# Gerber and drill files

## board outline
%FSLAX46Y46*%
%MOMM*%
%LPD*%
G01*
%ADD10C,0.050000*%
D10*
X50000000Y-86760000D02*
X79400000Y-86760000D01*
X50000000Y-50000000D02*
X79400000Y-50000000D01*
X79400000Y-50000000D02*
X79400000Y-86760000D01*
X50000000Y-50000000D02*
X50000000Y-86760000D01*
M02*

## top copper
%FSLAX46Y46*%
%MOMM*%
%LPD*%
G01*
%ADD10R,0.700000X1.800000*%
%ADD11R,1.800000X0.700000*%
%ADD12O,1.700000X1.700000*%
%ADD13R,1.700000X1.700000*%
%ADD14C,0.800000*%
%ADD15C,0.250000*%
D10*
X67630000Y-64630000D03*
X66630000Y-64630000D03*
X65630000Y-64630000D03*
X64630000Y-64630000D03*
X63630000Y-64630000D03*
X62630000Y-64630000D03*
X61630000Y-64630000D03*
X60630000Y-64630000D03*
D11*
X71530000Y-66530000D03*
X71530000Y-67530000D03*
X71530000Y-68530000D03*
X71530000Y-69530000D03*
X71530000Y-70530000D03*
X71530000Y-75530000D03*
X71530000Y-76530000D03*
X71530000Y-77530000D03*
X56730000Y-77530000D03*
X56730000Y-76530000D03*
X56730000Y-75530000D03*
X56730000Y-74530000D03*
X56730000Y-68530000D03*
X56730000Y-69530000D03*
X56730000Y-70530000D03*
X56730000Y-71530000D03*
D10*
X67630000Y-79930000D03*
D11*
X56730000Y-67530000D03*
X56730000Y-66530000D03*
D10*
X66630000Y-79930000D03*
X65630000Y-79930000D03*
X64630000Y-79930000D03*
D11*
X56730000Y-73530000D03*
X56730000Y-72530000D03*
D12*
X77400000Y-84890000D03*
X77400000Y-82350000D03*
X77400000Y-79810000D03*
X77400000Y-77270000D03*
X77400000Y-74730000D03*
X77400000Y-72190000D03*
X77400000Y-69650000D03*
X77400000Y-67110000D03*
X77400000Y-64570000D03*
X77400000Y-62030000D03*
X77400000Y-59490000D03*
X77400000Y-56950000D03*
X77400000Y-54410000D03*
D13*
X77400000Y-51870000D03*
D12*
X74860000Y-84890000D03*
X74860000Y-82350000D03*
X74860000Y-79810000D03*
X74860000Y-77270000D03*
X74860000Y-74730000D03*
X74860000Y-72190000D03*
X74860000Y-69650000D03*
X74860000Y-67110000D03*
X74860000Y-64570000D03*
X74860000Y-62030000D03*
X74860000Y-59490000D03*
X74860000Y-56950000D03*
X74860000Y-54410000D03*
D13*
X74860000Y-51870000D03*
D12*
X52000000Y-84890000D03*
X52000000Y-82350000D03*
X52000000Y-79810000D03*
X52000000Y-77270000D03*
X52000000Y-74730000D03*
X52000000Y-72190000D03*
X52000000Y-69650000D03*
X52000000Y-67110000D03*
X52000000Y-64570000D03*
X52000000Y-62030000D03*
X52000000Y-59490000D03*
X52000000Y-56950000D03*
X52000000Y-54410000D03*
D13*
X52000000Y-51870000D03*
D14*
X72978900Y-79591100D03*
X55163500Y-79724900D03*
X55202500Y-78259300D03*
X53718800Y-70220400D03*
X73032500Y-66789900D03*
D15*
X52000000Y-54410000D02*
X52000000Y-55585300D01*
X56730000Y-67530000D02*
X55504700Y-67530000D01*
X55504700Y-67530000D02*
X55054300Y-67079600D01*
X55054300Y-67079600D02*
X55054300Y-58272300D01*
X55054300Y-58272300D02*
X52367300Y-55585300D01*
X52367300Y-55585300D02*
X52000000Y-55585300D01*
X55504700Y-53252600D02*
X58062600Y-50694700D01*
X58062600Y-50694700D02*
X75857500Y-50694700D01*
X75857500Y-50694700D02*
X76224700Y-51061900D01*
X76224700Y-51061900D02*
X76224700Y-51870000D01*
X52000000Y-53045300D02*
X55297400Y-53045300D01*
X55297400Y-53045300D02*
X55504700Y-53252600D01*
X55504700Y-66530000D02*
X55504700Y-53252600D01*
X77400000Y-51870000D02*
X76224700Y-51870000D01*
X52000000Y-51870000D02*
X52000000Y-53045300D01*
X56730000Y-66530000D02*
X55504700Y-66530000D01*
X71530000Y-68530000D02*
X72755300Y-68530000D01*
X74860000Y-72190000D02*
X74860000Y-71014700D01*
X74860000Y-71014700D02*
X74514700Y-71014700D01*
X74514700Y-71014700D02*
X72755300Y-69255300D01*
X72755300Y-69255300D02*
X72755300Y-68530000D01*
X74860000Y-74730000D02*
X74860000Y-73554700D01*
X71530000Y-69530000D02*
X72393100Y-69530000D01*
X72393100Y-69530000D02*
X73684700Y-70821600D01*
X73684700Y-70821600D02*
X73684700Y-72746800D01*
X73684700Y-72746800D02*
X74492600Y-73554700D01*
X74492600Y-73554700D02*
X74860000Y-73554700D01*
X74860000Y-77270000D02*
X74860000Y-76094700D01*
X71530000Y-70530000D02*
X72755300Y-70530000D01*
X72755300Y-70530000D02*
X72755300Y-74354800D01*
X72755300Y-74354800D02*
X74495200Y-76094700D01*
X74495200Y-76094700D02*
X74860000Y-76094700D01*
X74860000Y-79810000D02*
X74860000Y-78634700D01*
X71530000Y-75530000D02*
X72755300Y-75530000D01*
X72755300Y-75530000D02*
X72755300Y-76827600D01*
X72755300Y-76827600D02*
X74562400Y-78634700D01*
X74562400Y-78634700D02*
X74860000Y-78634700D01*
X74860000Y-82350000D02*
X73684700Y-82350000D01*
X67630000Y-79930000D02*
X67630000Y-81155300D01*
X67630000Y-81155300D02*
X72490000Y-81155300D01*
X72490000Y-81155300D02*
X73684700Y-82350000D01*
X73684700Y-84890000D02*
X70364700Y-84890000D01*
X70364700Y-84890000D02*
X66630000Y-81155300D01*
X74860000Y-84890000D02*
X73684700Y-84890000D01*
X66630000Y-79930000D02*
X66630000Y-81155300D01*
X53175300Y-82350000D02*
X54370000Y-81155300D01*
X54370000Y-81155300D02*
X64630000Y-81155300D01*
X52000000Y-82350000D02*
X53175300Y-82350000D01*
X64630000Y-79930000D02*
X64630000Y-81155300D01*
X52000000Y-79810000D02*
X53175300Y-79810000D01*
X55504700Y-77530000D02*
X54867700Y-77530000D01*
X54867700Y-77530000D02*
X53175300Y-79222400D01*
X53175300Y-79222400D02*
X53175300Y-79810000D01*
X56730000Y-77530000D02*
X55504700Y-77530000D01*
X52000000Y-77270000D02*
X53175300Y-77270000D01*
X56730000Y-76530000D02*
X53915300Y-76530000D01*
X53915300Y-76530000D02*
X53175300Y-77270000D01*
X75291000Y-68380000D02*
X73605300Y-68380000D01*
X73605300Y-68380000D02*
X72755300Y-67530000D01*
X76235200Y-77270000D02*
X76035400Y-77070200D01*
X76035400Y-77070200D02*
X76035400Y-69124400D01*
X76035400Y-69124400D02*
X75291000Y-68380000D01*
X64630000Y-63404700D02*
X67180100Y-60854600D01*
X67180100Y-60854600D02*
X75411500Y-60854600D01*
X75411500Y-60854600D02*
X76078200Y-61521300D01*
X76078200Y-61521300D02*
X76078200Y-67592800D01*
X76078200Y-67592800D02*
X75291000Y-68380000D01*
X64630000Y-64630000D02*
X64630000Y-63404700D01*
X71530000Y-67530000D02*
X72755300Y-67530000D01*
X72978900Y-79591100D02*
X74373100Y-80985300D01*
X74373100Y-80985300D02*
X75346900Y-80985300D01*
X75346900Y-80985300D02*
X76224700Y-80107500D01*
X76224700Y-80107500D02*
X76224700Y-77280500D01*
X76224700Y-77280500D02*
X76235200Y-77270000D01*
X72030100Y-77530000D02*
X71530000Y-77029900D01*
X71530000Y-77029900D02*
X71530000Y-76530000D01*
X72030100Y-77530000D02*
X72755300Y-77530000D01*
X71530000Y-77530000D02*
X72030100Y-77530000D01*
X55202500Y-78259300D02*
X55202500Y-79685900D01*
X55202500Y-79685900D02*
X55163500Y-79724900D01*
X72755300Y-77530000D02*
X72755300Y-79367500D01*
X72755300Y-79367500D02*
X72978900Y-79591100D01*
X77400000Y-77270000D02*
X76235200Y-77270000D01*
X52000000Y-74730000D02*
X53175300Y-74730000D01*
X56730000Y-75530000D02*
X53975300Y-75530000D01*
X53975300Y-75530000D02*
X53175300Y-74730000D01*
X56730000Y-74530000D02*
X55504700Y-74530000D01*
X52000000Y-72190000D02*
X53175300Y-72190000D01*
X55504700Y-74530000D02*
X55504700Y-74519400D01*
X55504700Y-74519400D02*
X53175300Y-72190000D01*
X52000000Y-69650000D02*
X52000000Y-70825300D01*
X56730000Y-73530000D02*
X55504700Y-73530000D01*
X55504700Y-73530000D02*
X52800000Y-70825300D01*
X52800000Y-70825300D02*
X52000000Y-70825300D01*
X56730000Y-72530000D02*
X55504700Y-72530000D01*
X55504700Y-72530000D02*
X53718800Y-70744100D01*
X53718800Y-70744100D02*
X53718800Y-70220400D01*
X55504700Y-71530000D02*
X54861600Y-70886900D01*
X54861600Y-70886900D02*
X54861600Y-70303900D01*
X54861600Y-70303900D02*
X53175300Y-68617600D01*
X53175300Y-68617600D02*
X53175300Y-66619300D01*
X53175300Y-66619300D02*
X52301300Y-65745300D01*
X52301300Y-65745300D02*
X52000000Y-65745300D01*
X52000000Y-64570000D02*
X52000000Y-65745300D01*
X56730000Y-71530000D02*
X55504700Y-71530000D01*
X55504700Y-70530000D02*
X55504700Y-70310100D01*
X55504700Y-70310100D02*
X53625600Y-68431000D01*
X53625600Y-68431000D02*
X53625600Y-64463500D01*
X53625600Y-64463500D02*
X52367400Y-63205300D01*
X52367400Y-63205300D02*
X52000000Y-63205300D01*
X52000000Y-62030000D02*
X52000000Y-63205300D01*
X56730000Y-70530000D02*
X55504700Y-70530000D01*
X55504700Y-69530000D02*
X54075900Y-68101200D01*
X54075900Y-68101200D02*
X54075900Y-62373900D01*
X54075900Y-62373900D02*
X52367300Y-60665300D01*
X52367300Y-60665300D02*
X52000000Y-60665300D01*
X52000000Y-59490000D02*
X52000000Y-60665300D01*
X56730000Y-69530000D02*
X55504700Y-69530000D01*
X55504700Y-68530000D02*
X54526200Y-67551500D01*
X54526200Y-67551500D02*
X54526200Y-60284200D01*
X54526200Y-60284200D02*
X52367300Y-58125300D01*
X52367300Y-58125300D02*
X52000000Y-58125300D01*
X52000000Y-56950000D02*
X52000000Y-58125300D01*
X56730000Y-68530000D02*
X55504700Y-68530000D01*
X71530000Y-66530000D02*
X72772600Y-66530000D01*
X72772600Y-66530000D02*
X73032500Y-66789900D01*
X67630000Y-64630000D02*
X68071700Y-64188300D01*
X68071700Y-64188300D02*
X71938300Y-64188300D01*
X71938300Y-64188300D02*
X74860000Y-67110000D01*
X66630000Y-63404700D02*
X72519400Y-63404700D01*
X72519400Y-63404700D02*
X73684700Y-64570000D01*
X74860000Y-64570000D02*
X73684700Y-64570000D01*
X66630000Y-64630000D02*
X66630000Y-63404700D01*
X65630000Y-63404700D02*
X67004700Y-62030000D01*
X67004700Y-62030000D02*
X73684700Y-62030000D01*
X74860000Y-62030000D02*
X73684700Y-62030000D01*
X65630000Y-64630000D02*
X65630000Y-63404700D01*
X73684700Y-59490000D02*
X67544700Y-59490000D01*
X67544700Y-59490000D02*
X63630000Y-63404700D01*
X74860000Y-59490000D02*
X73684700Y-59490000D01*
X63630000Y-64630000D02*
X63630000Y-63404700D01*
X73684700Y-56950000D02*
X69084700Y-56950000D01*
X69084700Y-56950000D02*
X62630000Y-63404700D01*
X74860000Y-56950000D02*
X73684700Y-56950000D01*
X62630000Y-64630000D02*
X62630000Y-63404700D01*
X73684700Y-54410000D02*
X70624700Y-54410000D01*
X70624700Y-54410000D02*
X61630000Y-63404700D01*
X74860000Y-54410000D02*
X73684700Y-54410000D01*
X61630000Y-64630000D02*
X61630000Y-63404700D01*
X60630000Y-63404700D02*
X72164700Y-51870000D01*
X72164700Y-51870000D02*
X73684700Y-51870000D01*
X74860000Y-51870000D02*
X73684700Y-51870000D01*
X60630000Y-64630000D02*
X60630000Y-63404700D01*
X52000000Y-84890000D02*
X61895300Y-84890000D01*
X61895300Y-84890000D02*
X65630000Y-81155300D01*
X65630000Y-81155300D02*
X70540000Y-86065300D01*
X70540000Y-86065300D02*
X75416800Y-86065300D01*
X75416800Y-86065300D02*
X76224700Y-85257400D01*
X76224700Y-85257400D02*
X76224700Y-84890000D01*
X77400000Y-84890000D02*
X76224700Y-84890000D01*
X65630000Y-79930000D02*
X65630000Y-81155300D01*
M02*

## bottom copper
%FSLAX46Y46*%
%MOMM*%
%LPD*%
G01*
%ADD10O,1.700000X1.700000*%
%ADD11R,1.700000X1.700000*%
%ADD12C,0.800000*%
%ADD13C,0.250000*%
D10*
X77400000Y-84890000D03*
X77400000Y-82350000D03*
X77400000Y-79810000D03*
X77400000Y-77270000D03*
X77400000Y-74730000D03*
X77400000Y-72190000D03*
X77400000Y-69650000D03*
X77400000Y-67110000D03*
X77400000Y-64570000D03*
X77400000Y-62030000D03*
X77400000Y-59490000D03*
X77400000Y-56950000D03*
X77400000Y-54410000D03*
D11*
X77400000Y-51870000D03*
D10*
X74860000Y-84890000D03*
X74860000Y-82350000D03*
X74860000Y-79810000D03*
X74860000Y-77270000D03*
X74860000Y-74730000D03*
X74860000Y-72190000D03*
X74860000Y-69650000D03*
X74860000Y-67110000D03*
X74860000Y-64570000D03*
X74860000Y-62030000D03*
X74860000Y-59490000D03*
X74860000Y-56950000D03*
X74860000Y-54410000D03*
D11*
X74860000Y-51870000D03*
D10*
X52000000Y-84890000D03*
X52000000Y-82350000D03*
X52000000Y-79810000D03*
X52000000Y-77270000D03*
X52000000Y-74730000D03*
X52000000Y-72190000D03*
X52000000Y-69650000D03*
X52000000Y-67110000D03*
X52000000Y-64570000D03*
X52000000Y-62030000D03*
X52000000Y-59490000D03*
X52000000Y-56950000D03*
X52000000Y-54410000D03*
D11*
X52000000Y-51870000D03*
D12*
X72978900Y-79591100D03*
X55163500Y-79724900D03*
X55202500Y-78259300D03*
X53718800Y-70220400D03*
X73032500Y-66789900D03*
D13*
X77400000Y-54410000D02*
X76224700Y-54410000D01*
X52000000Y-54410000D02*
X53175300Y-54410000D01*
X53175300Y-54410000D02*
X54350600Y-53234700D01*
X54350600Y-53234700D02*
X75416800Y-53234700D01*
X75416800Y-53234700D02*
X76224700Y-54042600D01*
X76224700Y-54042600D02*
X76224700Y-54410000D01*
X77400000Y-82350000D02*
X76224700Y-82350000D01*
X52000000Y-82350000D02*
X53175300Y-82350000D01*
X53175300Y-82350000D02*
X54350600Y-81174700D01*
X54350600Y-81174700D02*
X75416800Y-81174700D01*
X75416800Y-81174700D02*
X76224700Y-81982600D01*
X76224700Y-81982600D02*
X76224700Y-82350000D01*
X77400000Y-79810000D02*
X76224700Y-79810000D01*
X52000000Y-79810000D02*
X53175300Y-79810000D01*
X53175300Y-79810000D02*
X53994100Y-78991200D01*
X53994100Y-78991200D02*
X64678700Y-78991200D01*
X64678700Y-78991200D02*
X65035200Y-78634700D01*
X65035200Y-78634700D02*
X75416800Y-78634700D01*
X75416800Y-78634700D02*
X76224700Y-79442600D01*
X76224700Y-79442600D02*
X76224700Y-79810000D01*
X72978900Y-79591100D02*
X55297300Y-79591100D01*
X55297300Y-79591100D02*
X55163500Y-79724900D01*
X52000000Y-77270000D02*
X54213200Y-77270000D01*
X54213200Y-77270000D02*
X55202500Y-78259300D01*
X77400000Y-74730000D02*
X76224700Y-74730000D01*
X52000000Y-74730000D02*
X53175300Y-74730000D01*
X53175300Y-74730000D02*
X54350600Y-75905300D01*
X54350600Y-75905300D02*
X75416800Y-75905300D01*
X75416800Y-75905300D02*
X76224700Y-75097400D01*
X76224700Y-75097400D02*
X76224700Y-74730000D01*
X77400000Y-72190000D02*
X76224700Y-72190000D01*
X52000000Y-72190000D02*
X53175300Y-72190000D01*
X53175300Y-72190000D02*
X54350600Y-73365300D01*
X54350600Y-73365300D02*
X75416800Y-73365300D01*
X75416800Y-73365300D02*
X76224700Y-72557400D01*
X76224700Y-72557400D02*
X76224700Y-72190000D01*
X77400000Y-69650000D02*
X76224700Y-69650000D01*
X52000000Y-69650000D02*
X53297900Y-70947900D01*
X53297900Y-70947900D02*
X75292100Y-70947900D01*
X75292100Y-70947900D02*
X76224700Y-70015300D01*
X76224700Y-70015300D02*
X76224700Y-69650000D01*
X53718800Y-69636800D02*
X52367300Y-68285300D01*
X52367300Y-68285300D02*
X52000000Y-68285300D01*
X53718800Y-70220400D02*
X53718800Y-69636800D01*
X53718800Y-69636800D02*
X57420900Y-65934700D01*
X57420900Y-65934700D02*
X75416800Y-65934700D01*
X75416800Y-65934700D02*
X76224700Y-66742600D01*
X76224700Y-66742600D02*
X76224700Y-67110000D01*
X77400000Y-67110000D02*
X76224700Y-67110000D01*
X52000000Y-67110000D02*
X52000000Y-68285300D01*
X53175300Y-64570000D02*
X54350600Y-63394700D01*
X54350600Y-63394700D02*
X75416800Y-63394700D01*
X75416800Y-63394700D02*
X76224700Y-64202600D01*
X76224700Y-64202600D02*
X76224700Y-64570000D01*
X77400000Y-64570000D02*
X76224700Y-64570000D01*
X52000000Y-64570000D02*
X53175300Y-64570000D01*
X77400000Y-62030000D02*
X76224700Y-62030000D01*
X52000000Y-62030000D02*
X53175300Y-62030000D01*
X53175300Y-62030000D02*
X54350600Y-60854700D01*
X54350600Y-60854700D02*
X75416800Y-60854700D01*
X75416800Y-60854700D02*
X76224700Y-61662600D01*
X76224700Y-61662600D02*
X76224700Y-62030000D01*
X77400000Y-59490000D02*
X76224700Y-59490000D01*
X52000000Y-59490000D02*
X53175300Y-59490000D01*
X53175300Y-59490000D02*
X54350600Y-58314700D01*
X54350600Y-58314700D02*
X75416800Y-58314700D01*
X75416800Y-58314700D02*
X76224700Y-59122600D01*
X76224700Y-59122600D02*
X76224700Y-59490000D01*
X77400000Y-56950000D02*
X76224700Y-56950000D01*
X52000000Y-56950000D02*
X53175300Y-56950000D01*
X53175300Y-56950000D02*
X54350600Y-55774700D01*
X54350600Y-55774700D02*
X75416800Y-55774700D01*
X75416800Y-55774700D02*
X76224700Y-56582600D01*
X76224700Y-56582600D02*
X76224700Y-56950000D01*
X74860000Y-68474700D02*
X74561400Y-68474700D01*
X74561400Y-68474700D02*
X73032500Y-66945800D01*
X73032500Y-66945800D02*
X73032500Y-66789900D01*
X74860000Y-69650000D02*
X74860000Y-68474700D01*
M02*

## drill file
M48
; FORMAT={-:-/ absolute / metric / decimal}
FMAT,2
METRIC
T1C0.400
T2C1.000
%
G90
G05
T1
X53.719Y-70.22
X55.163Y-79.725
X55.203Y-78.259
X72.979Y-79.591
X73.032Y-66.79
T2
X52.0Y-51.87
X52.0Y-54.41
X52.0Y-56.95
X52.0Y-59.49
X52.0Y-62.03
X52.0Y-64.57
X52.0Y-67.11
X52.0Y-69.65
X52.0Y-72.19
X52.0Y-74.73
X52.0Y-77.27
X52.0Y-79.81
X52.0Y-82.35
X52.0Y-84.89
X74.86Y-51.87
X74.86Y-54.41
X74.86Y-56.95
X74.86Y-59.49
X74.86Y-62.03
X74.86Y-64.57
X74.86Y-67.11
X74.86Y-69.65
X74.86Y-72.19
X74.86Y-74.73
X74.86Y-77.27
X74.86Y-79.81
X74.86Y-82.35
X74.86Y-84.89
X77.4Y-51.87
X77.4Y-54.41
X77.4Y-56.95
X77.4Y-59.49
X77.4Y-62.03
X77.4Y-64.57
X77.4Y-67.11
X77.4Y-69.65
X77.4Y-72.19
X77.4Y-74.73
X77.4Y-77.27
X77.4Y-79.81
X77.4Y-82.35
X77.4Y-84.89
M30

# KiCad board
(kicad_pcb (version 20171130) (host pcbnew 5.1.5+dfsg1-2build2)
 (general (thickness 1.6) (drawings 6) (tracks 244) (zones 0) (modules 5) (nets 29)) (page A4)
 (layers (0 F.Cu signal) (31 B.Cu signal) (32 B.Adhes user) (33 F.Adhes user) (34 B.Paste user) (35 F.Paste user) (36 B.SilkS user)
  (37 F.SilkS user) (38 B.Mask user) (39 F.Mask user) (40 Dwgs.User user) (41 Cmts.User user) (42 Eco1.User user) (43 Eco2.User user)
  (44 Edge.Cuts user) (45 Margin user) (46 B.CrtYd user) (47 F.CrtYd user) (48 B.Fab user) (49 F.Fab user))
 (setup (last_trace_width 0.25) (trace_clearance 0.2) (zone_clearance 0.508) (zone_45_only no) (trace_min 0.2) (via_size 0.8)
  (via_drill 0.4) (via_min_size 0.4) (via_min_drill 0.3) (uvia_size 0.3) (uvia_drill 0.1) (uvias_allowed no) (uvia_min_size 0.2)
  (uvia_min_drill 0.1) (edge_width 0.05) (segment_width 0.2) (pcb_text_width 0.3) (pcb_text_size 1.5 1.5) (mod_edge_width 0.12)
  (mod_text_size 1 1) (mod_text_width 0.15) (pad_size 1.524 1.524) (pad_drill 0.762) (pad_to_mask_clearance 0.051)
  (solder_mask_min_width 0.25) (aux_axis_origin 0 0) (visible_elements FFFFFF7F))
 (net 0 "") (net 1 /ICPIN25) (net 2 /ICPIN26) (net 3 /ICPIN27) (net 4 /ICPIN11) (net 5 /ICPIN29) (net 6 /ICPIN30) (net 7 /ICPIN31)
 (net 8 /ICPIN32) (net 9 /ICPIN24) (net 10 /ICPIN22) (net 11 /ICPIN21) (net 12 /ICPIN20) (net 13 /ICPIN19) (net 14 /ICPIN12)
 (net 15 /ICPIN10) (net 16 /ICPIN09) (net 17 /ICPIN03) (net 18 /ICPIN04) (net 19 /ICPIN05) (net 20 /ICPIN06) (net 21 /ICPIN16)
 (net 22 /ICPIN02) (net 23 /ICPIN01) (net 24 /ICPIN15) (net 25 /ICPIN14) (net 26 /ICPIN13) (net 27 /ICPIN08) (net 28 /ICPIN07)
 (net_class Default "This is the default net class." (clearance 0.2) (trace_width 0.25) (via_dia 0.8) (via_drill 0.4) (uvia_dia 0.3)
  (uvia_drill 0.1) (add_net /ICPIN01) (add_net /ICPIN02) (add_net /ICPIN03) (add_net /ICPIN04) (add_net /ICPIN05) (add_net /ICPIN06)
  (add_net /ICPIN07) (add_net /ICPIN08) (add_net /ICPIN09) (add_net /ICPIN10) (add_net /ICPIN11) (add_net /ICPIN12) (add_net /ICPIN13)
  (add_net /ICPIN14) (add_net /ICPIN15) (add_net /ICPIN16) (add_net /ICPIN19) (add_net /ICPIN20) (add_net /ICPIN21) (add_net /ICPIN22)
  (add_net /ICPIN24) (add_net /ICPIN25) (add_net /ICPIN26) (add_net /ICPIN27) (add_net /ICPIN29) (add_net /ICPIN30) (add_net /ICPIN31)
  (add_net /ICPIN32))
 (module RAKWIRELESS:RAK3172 (layer F.Cu) (at 64.13 72.28)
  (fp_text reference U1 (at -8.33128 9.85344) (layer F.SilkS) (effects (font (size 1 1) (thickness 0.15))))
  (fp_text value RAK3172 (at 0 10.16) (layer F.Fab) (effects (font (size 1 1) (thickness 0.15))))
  (pad 25 smd rect (at 3.5 -7.65 270) (size 1.8 0.7) (layers F.Cu F.Paste F.Mask) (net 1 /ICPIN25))
  (pad 26 smd rect (at 2.5 -7.65 270) (size 1.8 0.7) (layers F.Cu F.Paste F.Mask) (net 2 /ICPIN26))
  (pad 27 smd rect (at 1.5 -7.65 270) (size 1.8 0.7) (layers F.Cu F.Paste F.Mask) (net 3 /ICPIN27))
  (pad 28 smd rect (at 0.5 -7.65 270) (size 1.8 0.7) (layers F.Cu F.Paste F.Mask) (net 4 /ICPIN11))
  (pad 29 smd rect (at -0.5 -7.65 270) (size 1.8 0.7) (layers F.Cu F.Paste F.Mask) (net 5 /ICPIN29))
  (pad 30 smd rect (at -1.5 -7.65 270) (size 1.8 0.7) (layers F.Cu F.Paste F.Mask) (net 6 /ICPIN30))
  (pad 31 smd rect (at -2.5 -7.65 270) (size 1.8 0.7) (layers F.Cu F.Paste F.Mask) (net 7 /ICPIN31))
  (pad 32 smd rect (at -3.5 -7.65 270) (size 1.8 0.7) (layers F.Cu F.Paste F.Mask) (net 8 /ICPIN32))
  (pad 24 smd rect (at 7.4 -5.75) (size 1.8 0.7) (layers F.Cu F.Paste F.Mask) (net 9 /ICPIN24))
  (pad 23 smd rect (at 7.4 -4.75) (size 1.8 0.7) (layers F.Cu F.Paste F.Mask) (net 4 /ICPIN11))
  (pad 22 smd rect (at 7.4 -3.75) (size 1.8 0.7) (layers F.Cu F.Paste F.Mask) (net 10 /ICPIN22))
  (pad 21 smd rect (at 7.4 -2.75) (size 1.8 0.7) (layers F.Cu F.Paste F.Mask) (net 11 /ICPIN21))
  (pad 20 smd rect (at 7.4 -1.75) (size 1.8 0.7) (layers F.Cu F.Paste F.Mask) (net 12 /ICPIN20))
  (pad 19 smd rect (at 7.4 3.25) (size 1.8 0.7) (layers F.Cu F.Paste F.Mask) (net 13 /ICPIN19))
  (pad 18 smd rect (at 7.4 4.25) (size 1.8 0.7) (layers F.Cu F.Paste F.Mask) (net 4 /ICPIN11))
  (pad 17 smd rect (at 7.4 5.25) (size 1.8 0.7) (layers F.Cu F.Paste F.Mask) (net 4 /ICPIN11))
  (pad 12 smd rect (at -7.4 5.25) (size 1.8 0.7) (layers F.Cu F.Paste F.Mask) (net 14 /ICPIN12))
  (pad 11 smd rect (at -7.4 4.25) (size 1.8 0.7) (layers F.Cu F.Paste F.Mask) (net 4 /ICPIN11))
  (pad 10 smd rect (at -7.4 3.25) (size 1.8 0.7) (layers F.Cu F.Paste F.Mask) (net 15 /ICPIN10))
  (pad 9 smd rect (at -7.4 2.25) (size 1.8 0.7) (layers F.Cu F.Paste F.Mask) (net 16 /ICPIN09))
  (pad 3 smd rect (at -7.4 -3.75) (size 1.8 0.7) (layers F.Cu F.Paste F.Mask) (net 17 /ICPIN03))
  (pad 4 smd rect (at -7.4 -2.75) (size 1.8 0.7) (layers F.Cu F.Paste F.Mask) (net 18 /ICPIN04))
  (pad 5 smd rect (at -7.4 -1.75) (size 1.8 0.7) (layers F.Cu F.Paste F.Mask) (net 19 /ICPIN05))
  (pad 6 smd rect (at -7.4 -0.75) (size 1.8 0.7) (layers F.Cu F.Paste F.Mask) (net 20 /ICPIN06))
  (pad 16 smd rect (at 3.5 7.65 90) (size 1.8 0.7) (layers F.Cu F.Paste F.Mask) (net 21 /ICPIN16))
  (pad 2 smd rect (at -7.4 -4.75) (size 1.8 0.7) (layers F.Cu F.Paste F.Mask) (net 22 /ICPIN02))
  (pad 1 smd rect (at -7.4 -5.75) (size 1.8 0.7) (layers F.Cu F.Paste F.Mask) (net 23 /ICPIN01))
  (pad 15 smd rect (at 2.5 7.65 90) (size 1.8 0.7) (layers F.Cu F.Paste F.Mask) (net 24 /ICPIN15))
  (pad 14 smd rect (at 1.5 7.65 90) (size 1.8 0.7) (layers F.Cu F.Paste F.Mask) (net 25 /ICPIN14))
  (pad 13 smd rect (at 0.5 7.65 270) (size 1.8 0.7) (layers F.Cu F.Paste F.Mask) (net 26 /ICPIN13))
  (pad 8 smd rect (at -7.4 1.25) (size 1.8 0.7) (layers F.Cu F.Paste F.Mask) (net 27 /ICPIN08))
  (pad 7 smd rect (at -7.4 0.25) (size 1.8 0.7) (layers F.Cu F.Paste F.Mask) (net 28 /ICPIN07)))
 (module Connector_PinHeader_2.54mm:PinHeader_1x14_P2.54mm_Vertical (layer F.Cu) (at 77.4 51.87)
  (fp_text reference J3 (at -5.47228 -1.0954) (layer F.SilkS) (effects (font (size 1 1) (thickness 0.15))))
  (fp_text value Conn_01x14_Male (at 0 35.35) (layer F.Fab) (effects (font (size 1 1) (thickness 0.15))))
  (pad 14 thru_hole oval (at 0 33.02) (size 1.7 1.7) (drill 1) (layers *.Cu *.Mask) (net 25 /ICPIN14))
  (pad 13 thru_hole oval (at 0 30.48) (size 1.7 1.7) (drill 1) (layers *.Cu *.Mask) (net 26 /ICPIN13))
  (pad 12 thru_hole oval (at 0 27.94) (size 1.7 1.7) (drill 1) (layers *.Cu *.Mask) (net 14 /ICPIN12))
  (pad 11 thru_hole oval (at 0 25.4) (size 1.7 1.7) (drill 1) (layers *.Cu *.Mask) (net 4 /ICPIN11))
  (pad 10 thru_hole oval (at 0 22.86) (size 1.7 1.7) (drill 1) (layers *.Cu *.Mask) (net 15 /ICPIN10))
  (pad 9 thru_hole oval (at 0 20.32) (size 1.7 1.7) (drill 1) (layers *.Cu *.Mask) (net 16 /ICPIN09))
  (pad 8 thru_hole oval (at 0 17.78) (size 1.7 1.7) (drill 1) (layers *.Cu *.Mask) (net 27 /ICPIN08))
  (pad 7 thru_hole oval (at 0 15.24) (size 1.7 1.7) (drill 1) (layers *.Cu *.Mask) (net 28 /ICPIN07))
  (pad 6 thru_hole oval (at 0 12.7) (size 1.7 1.7) (drill 1) (layers *.Cu *.Mask) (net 20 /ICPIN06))
  (pad 5 thru_hole oval (at 0 10.16) (size 1.7 1.7) (drill 1) (layers *.Cu *.Mask) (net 19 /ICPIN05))
  (pad 4 thru_hole oval (at 0 7.62) (size 1.7 1.7) (drill 1) (layers *.Cu *.Mask) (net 18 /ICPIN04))
  (pad 3 thru_hole oval (at 0 5.08) (size 1.7 1.7) (drill 1) (layers *.Cu *.Mask) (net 17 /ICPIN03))
  (pad 2 thru_hole oval (at 0 2.54) (size 1.7 1.7) (drill 1) (layers *.Cu *.Mask) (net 22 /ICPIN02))
  (pad 1 thru_hole rect (at 0 0) (size 1.7 1.7) (drill 1) (layers *.Cu *.Mask) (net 23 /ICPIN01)))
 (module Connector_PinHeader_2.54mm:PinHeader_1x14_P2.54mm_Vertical (layer F.Cu) (at 74.86 51.87)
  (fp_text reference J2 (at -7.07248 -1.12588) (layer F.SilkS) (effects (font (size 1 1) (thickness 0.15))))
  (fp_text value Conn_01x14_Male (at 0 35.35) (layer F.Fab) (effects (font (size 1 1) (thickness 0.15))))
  (pad 14 thru_hole oval (at 0 33.02) (size 1.7 1.7) (drill 1) (layers *.Cu *.Mask) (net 24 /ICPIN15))
  (pad 13 thru_hole oval (at 0 30.48) (size 1.7 1.7) (drill 1) (layers *.Cu *.Mask) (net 21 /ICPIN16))
  (pad 12 thru_hole oval (at 0 27.94) (size 1.7 1.7) (drill 1) (layers *.Cu *.Mask) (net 13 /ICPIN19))
  (pad 11 thru_hole oval (at 0 25.4) (size 1.7 1.7) (drill 1) (layers *.Cu *.Mask) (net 12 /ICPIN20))
  (pad 10 thru_hole oval (at 0 22.86) (size 1.7 1.7) (drill 1) (layers *.Cu *.Mask) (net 11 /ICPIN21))
  (pad 9 thru_hole oval (at 0 20.32) (size 1.7 1.7) (drill 1) (layers *.Cu *.Mask) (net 10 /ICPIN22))
  (pad 8 thru_hole oval (at 0 17.78) (size 1.7 1.7) (drill 1) (layers *.Cu *.Mask) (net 9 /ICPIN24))
  (pad 7 thru_hole oval (at 0 15.24) (size 1.7 1.7) (drill 1) (layers *.Cu *.Mask) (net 1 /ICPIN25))
  (pad 6 thru_hole oval (at 0 12.7) (size 1.7 1.7) (drill 1) (layers *.Cu *.Mask) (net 2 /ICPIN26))
  (pad 5 thru_hole oval (at 0 10.16) (size 1.7 1.7) (drill 1) (layers *.Cu *.Mask) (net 3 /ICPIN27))
  (pad 4 thru_hole oval (at 0 7.62) (size 1.7 1.7) (drill 1) (layers *.Cu *.Mask) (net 5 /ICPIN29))
  (pad 3 thru_hole oval (at 0 5.08) (size 1.7 1.7) (drill 1) (layers *.Cu *.Mask) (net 6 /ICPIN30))
  (pad 2 thru_hole oval (at 0 2.54) (size 1.7 1.7) (drill 1) (layers *.Cu *.Mask) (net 7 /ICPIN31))
  (pad 1 thru_hole rect (at 0 0) (size 1.7 1.7) (drill 1) (layers *.Cu *.Mask) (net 8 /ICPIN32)))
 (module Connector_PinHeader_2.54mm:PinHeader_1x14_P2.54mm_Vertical (layer F.Cu) (at 52 51.87)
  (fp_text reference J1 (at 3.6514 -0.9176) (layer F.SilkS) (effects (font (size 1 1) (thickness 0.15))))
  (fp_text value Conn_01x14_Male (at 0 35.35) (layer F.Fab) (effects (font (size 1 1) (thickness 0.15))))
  (pad 14 thru_hole oval (at 0 33.02) (size 1.7 1.7) (drill 1) (layers *.Cu *.Mask) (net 25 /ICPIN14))
  (pad 13 thru_hole oval (at 0 30.48) (size 1.7 1.7) (drill 1) (layers *.Cu *.Mask) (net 26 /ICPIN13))
  (pad 12 thru_hole oval (at 0 27.94) (size 1.7 1.7) (drill 1) (layers *.Cu *.Mask) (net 14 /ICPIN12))
  (pad 11 thru_hole oval (at 0 25.4) (size 1.7 1.7) (drill 1) (layers *.Cu *.Mask) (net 4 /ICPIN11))
  (pad 10 thru_hole oval (at 0 22.86) (size 1.7 1.7) (drill 1) (layers *.Cu *.Mask) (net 15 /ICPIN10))
  (pad 9 thru_hole oval (at 0 20.32) (size 1.7 1.7) (drill 1) (layers *.Cu *.Mask) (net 16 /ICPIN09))
  (pad 8 thru_hole oval (at 0 17.78) (size 1.7 1.7) (drill 1) (layers *.Cu *.Mask) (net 27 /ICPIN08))
  (pad 7 thru_hole oval (at 0 15.24) (size 1.7 1.7) (drill 1) (layers *.Cu *.Mask) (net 28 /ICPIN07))
  (pad 6 thru_hole oval (at 0 12.7) (size 1.7 1.7) (drill 1) (layers *.Cu *.Mask) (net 20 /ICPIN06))
  (pad 5 thru_hole oval (at 0 10.16) (size 1.7 1.7) (drill 1) (layers *.Cu *.Mask) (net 19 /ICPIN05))
  (pad 4 thru_hole oval (at 0 7.62) (size 1.7 1.7) (drill 1) (layers *.Cu *.Mask) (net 18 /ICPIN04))
  (pad 3 thru_hole oval (at 0 5.08) (size 1.7 1.7) (drill 1) (layers *.Cu *.Mask) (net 17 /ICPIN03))
  (pad 2 thru_hole oval (at 0 2.54) (size 1.7 1.7) (drill 1) (layers *.Cu *.Mask) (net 22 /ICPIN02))
  (pad 1 thru_hole rect (at 0 0) (size 1.7 1.7) (drill 1) (layers *.Cu *.Mask) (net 23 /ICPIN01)))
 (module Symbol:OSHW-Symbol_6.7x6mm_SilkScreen (layer F.Cu) (at 62.17412 53.67528)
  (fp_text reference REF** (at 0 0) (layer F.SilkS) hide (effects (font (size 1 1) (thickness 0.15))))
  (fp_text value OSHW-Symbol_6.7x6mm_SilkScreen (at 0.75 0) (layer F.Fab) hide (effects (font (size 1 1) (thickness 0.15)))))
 (gr_line (start 50 86.76) (end 79.4 86.76) (layer Edge.Cuts) (width 0.05))
 (gr_line (start 50 50) (end 79.4 50) (layer Edge.Cuts) (width 0.05))
 (gr_line (start 79.4 50) (end 79.4 86.76) (layer Edge.Cuts) (width 0.05))
 (gr_line (start 50 50) (end 50 86.76) (layer Edge.Cuts) (width 0.05))
 (segment (start 52 54.41) (end 52 55.5853) (width 0.25) (layer F.Cu) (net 22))
 (segment (start 56.73 67.53) (end 55.5047 67.53) (width 0.25) (layer F.Cu) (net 22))
 (segment (start 55.5047 67.53) (end 55.0543 67.0796) (width 0.25) (layer F.Cu) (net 22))
 (segment (start 55.0543 67.0796) (end 55.0543 58.2723) (width 0.25) (layer F.Cu) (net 22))
 (segment (start 55.0543 58.2723) (end 52.3673 55.5853) (width 0.25) (layer F.Cu) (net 22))
 (segment (start 52.3673 55.5853) (end 52 55.5853) (width 0.25) (layer F.Cu) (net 22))
 (segment (start 77.4 54.41) (end 76.2247 54.41) (width 0.25) (layer B.Cu) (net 22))
 (segment (start 52 54.41) (end 53.1753 54.41) (width 0.25) (layer B.Cu) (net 22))
 (segment (start 53.1753 54.41) (end 54.3506 53.2347) (width 0.25) (layer B.Cu) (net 22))
 (segment (start 54.3506 53.2347) (end 75.4168 53.2347) (width 0.25) (layer B.Cu) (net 22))
 (segment (start 75.4168 53.2347) (end 76.2247 54.0426) (width 0.25) (layer B.Cu) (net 22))
 (segment (start 76.2247 54.0426) (end 76.2247 54.41) (width 0.25) (layer B.Cu) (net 22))
 (segment (start 55.5047 53.2526) (end 58.0626 50.6947) (width 0.25) (layer F.Cu) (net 23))
 (segment (start 58.0626 50.6947) (end 75.8575 50.6947) (width 0.25) (layer F.Cu) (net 23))
 (segment (start 75.8575 50.6947) (end 76.2247 51.0619) (width 0.25) (layer F.Cu) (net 23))
 (segment (start 76.2247 51.0619) (end 76.2247 51.87) (width 0.25) (layer F.Cu) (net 23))
 (segment (start 52 53.0453) (end 55.2974 53.0453) (width 0.25) (layer F.Cu) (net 23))
 (segment (start 55.2974 53.0453) (end 55.5047 53.2526) (width 0.25) (layer F.Cu) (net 23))
 (segment (start 55.5047 66.53) (end 55.5047 53.2526) (width 0.25) (layer F.Cu) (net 23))
 (segment (start 77.4 51.87) (end 76.2247 51.87) (width 0.25) (layer F.Cu) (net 23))
 (segment (start 52 51.87) (end 52 53.0453) (width 0.25) (layer F.Cu) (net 23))
 (segment (start 56.73 66.53) (end 55.5047 66.53) (width 0.25) (layer F.Cu) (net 23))
 (segment (start 71.53 68.53) (end 72.7553 68.53) (width 0.25) (layer F.Cu) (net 10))
 (segment (start 74.86 72.19) (end 74.86 71.0147) (width 0.25) (layer F.Cu) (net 10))
 (segment (start 74.86 71.0147) (end 74.5147 71.0147) (width 0.25) (layer F.Cu) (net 10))
 (segment (start 74.5147 71.0147) (end 72.7553 69.2553) (width 0.25) (layer F.Cu) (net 10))
 (segment (start 72.7553 69.2553) (end 72.7553 68.53) (width 0.25) (layer F.Cu) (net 10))
 (segment (start 74.86 74.73) (end 74.86 73.5547) (width 0.25) (layer F.Cu) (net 11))
 (segment (start 71.53 69.53) (end 72.3931 69.53) (width 0.25) (layer F.Cu) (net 11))
 (segment (start 72.3931 69.53) (end 73.6847 70.8216) (width 0.25) (layer F.Cu) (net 11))
 (segment (start 73.6847 70.8216) (end 73.6847 72.7468) (width 0.25) (layer F.Cu) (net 11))
 (segment (start 73.6847 72.7468) (end 74.4926 73.5547) (width 0.25) (layer F.Cu) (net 11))
 (segment (start 74.4926 73.5547) (end 74.86 73.5547) (width 0.25) (layer F.Cu) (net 11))
 (segment (start 74.86 77.27) (end 74.86 76.0947) (width 0.25) (layer F.Cu) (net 12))
 (segment (start 71.53 70.53) (end 72.7553 70.53) (width 0.25) (layer F.Cu) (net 12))
 (segment (start 72.7553 70.53) (end 72.7553 74.3548) (width 0.25) (layer F.Cu) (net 12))
 (segment (start 72.7553 74.3548) (end 74.4952 76.0947) (width 0.25) (layer F.Cu) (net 12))
 (segment (start 74.4952 76.0947) (end 74.86 76.0947) (width 0.25) (layer F.Cu) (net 12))
 (segment (start 74.86 79.81) (end 74.86 78.6347) (width 0.25) (layer F.Cu) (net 13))
 (segment (start 71.53 75.53) (end 72.7553 75.53) (width 0.25) (layer F.Cu) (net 13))
 (segment (start 72.7553 75.53) (end 72.7553 76.8276) (width 0.25) (layer F.Cu) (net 13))
 (segment (start 72.7553 76.8276) (end 74.5624 78.6347) (width 0.25) (layer F.Cu) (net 13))
 (segment (start 74.5624 78.6347) (end 74.86 78.6347) (width 0.25) (layer F.Cu) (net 13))
 (segment (start 74.86 82.35) (end 73.6847 82.35) (width 0.25) (layer F.Cu) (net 21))
 (segment (start 67.63 79.93) (end 67.63 81.1553) (width 0.25) (layer F.Cu) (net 21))
 (segment (start 67.63 81.1553) (end 72.49 81.1553) (width 0.25) (layer F.Cu) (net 21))
 (segment (start 72.49 81.1553) (end 73.6847 82.35) (width 0.25) (layer F.Cu) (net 21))
 (segment (start 73.6847 84.89) (end 70.3647 84.89) (width 0.25) (layer F.Cu) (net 24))
 (segment (start 70.3647 84.89) (end 66.63 81.1553) (width 0.25) (layer F.Cu) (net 24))
 (segment (start 74.86 84.89) (end 73.6847 84.89) (width 0.25) (layer F.Cu) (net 24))
 (segment (start 66.63 79.93) (end 66.63 81.1553) (width 0.25) (layer F.Cu) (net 24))
 (segment (start 77.4 82.35) (end 76.2247 82.35) (width 0.25) (layer B.Cu) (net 26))
 (segment (start 52 82.35) (end 53.1753 82.35) (width 0.25) (layer B.Cu) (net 26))
 (segment (start 53.1753 82.35) (end 54.3506 81.1747) (width 0.25) (layer B.Cu) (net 26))
 (segment (start 54.3506 81.1747) (end 75.4168 81.1747) (width 0.25) (layer B.Cu) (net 26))
 (segment (start 75.4168 81.1747) (end 76.2247 81.9826) (width 0.25) (layer B.Cu) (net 26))
 (segment (start 76.2247 81.9826) (end 76.2247 82.35) (width 0.25) (layer B.Cu) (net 26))
 (segment (start 53.1753 82.35) (end 54.37 81.1553) (width 0.25) (layer F.Cu) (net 26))
 (segment (start 54.37 81.1553) (end 64.63 81.1553) (width 0.25) (layer F.Cu) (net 26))
 (segment (start 52 82.35) (end 53.1753 82.35) (width 0.25) (layer F.Cu) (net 26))
 (segment (start 64.63 79.93) (end 64.63 81.1553) (width 0.25) (layer F.Cu) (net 26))
 (segment (start 77.4 79.81) (end 76.2247 79.81) (width 0.25) (layer B.Cu) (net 14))
 (segment (start 52 79.81) (end 53.1753 79.81) (width 0.25) (layer B.Cu) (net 14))
 (segment (start 53.1753 79.81) (end 53.9941 78.9912) (width 0.25) (layer B.Cu) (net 14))
 (segment (start 53.9941 78.9912) (end 64.6787 78.9912) (width 0.25) (layer B.Cu) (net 14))
 (segment (start 64.6787 78.9912) (end 65.0352 78.6347) (width 0.25) (layer B.Cu) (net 14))
 (segment (start 65.0352 78.6347) (end 75.4168 78.6347) (width 0.25) (layer B.Cu) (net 14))
 (segment (start 75.4168 78.6347) (end 76.2247 79.4426) (width 0.25) (layer B.Cu) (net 14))
 (segment (start 76.2247 79.4426) (end 76.2247 79.81) (width 0.25) (layer B.Cu) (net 14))
 (segment (start 52 79.81) (end 53.1753 79.81) (width 0.25) (layer F.Cu) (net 14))
 (segment (start 55.5047 77.53) (end 54.8677 77.53) (width 0.25) (layer F.Cu) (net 14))
 (segment (start 54.8677 77.53) (end 53.1753 79.2224) (width 0.25) (layer F.Cu) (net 14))
 (segment (start 53.1753 79.2224) (end 53.1753 79.81) (width 0.25) (layer F.Cu) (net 14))
 (segment (start 56.73 77.53) (end 55.5047 77.53) (width 0.25) (layer F.Cu) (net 14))
 (segment (start 52 77.27) (end 53.1753 77.27) (width 0.25) (layer F.Cu) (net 4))
 (segment (start 56.73 76.53) (end 53.9153 76.53) (width 0.25) (layer F.Cu) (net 4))
 (segment (start 53.9153 76.53) (end 53.1753 77.27) (width 0.25) (layer F.Cu) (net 4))
 (segment (start 75.291 68.38) (end 73.6053 68.38) (width 0.25) (layer F.Cu) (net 4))
 (segment (start 73.6053 68.38) (end 72.7553 67.53) (width 0.25) (layer F.Cu) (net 4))
 (segment (start 76.2352 77.27) (end 76.0354 77.0702) (width 0.25) (layer F.Cu) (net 4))
 (segment (start 76.0354 77.0702) (end 76.0354 69.1244) (width 0.25) (layer F.Cu) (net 4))
 (segment (start 76.0354 69.1244) (end 75.291 68.38) (width 0.25) (layer F.Cu) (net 4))
 (segment (start 64.63 63.4047) (end 67.1801 60.8546) (width 0.25) (layer F.Cu) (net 4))
 (segment (start 67.1801 60.8546) (end 75.4115 60.8546) (width 0.25) (layer F.Cu) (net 4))
 (segment (start 75.4115 60.8546) (end 76.0782 61.5213) (width 0.25) (layer F.Cu) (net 4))
 (segment (start 76.0782 61.5213) (end 76.0782 67.5928) (width 0.25) (layer F.Cu) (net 4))
 (segment (start 76.0782 67.5928) (end 75.291 68.38) (width 0.25) (layer F.Cu) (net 4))
 (segment (start 64.63 64.63) (end 64.63 63.4047) (width 0.25) (layer F.Cu) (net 4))
 (segment (start 71.53 67.53) (end 72.7553 67.53) (width 0.25) (layer F.Cu) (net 4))
 (segment (start 72.9789 79.5911) (end 74.3731 80.9853) (width 0.25) (layer F.Cu) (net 4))
 (segment (start 74.3731 80.9853) (end 75.3469 80.9853) (width 0.25) (layer F.Cu) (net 4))
 (segment (start 75.3469 80.9853) (end 76.2247 80.1075) (width 0.25) (layer F.Cu) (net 4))
 (segment (start 76.2247 80.1075) (end 76.2247 77.2805) (width 0.25) (layer F.Cu) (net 4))
 (segment (start 76.2247 77.2805) (end 76.2352 77.27) (width 0.25) (layer F.Cu) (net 4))
 (segment (start 72.0301 77.53) (end 71.53 77.0299) (width 0.25) (layer F.Cu) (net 4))
 (segment (start 71.53 77.0299) (end 71.53 76.53) (width 0.25) (layer F.Cu) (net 4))
 (segment (start 72.0301 77.53) (end 72.7553 77.53) (width 0.25) (layer F.Cu) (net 4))
 (segment (start 71.53 77.53) (end 72.0301 77.53) (width 0.25) (layer F.Cu) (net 4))
 (segment (start 55.2025 78.2593) (end 55.2025 79.6859) (width 0.25) (layer F.Cu) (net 4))
 (segment (start 55.2025 79.6859) (end 55.1635 79.7249) (width 0.25) (layer F.Cu) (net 4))
 (segment (start 72.9789 79.5911) (end 55.2973 79.5911) (width 0.25) (layer B.Cu) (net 4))
 (segment (start 55.2973 79.5911) (end 55.1635 79.7249) (width 0.25) (layer B.Cu) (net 4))
 (segment (start 72.7553 77.53) (end 72.7553 79.3675) (width 0.25) (layer F.Cu) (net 4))
 (segment (start 72.7553 79.3675) (end 72.9789 79.5911) (width 0.25) (layer F.Cu) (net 4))
 (segment (start 52 77.27) (end 54.2132 77.27) (width 0.25) (layer B.Cu) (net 4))
 (segment (start 54.2132 77.27) (end 55.2025 78.2593) (width 0.25) (layer B.Cu) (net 4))
 (segment (start 77.4 77.27) (end 76.2352 77.27) (width 0.25) (layer F.Cu) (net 4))
 (via (at 72.9789 79.5911) (size 0.8) (layers F.Cu B.Cu) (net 4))
 (via (at 55.1635 79.7249) (size 0.8) (layers F.Cu B.Cu) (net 4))
 (via (at 55.2025 78.2593) (size 0.8) (layers F.Cu B.Cu) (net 4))
 (segment (start 52 74.73) (end 53.1753 74.73) (width 0.25) (layer F.Cu) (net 15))
 (segment (start 56.73 75.53) (end 53.9753 75.53) (width 0.25) (layer F.Cu) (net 15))
 (segment (start 53.9753 75.53) (end 53.1753 74.73) (width 0.25) (layer F.Cu) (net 15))
 (segment (start 77.4 74.73) (end 76.2247 74.73) (width 0.25) (layer B.Cu) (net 15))
 (segment (start 52 74.73) (end 53.1753 74.73) (width 0.25) (layer B.Cu) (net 15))
 (segment (start 53.1753 74.73) (end 54.3506 75.9053) (width 0.25) (layer B.Cu) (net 15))
 (segment (start 54.3506 75.9053) (end 75.4168 75.9053) (width 0.25) (layer B.Cu) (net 15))
 (segment (start 75.4168 75.9053) (end 76.2247 75.0974) (width 0.25) (layer B.Cu) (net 15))
 (segment (start 76.2247 75.0974) (end 76.2247 74.73) (width 0.25) (layer B.Cu) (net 15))
 (segment (start 77.4 72.19) (end 76.2247 72.19) (width 0.25) (layer B.Cu) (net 16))
 (segment (start 52 72.19) (end 53.1753 72.19) (width 0.25) (layer B.Cu) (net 16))
 (segment (start 53.1753 72.19) (end 54.3506 73.3653) (width 0.25) (layer B.Cu) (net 16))
 (segment (start 54.3506 73.3653) (end 75.4168 73.3653) (width 0.25) (layer B.Cu) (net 16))
 (segment (start 75.4168 73.3653) (end 76.2247 72.5574) (width 0.25) (layer B.Cu) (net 16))
 (segment (start 76.2247 72.5574) (end 76.2247 72.19) (width 0.25) (layer B.Cu) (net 16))
 (segment (start 56.73 74.53) (end 55.5047 74.53) (width 0.25) (layer F.Cu) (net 16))
 (segment (start 52 72.19) (end 53.1753 72.19) (width 0.25) (layer F.Cu) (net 16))
 (segment (start 55.5047 74.53) (end 55.5047 74.5194) (width 0.25) (layer F.Cu) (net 16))
 (segment (start 55.5047 74.5194) (end 53.1753 72.19) (width 0.25) (layer F.Cu) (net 16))
 (segment (start 77.4 69.65) (end 76.2247 69.65) (width 0.25) (layer B.Cu) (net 27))
 (segment (start 52 69.65) (end 53.2979 70.9479) (width 0.25) (layer B.Cu) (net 27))
 (segment (start 53.2979 70.9479) (end 75.2921 70.9479) (width 0.25) (layer B.Cu) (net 27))
 (segment (start 75.2921 70.9479) (end 76.2247 70.0153) (width 0.25) (layer B.Cu) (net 27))
 (segment (start 76.2247 70.0153) (end 76.2247 69.65) (width 0.25) (layer B.Cu) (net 27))
 (segment (start 52 69.65) (end 52 70.8253) (width 0.25) (layer F.Cu) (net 27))
 (segment (start 56.73 73.53) (end 55.5047 73.53) (width 0.25) (layer F.Cu) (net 27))
 (segment (start 55.5047 73.53) (end 52.8 70.8253) (width 0.25) (layer F.Cu) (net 27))
 (segment (start 52.8 70.8253) (end 52 70.8253) (width 0.25) (layer F.Cu) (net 27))
 (segment (start 53.7188 69.6368) (end 52.3673 68.2853) (width 0.25) (layer B.Cu) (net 28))
 (segment (start 52.3673 68.2853) (end 52 68.2853) (width 0.25) (layer B.Cu) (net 28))
 (segment (start 53.7188 70.2204) (end 53.7188 69.6368) (width 0.25) (layer B.Cu) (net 28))
 (segment (start 53.7188 69.6368) (end 57.4209 65.9347) (width 0.25) (layer B.Cu) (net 28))
 (segment (start 57.4209 65.9347) (end 75.4168 65.9347) (width 0.25) (layer B.Cu) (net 28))
 (segment (start 75.4168 65.9347) (end 76.2247 66.7426) (width 0.25) (layer B.Cu) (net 28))
 (segment (start 76.2247 66.7426) (end 76.2247 67.11) (width 0.25) (layer B.Cu) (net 28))
 (segment (start 77.4 67.11) (end 76.2247 67.11) (width 0.25) (layer B.Cu) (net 28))
 (segment (start 56.73 72.53) (end 55.5047 72.53) (width 0.25) (layer F.Cu) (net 28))
 (segment (start 52 67.11) (end 52 68.2853) (width 0.25) (layer B.Cu) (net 28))
 (segment (start 55.5047 72.53) (end 53.7188 70.7441) (width 0.25) (layer F.Cu) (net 28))
 (segment (start 53.7188 70.7441) (end 53.7188 70.2204) (width 0.25) (layer F.Cu) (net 28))
 (via (at 53.7188 70.2204) (size 0.8) (layers F.Cu B.Cu) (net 28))
 (segment (start 55.5047 71.53) (end 54.8616 70.8869) (width 0.25) (layer F.Cu) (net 20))
 (segment (start 54.8616 70.8869) (end 54.8616 70.3039) (width 0.25) (layer F.Cu) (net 20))
 (segment (start 54.8616 70.3039) (end 53.1753 68.6176) (width 0.25) (layer F.Cu) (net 20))
 (segment (start 53.1753 68.6176) (end 53.1753 66.6193) (width 0.25) (layer F.Cu) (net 20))
 (segment (start 53.1753 66.6193) (end 52.3013 65.7453) (width 0.25) (layer F.Cu) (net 20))
 (segment (start 52.3013 65.7453) (end 52 65.7453) (width 0.25) (layer F.Cu) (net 20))
 (segment (start 53.1753 64.57) (end 54.3506 63.3947) (width 0.25) (layer B.Cu) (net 20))
 (segment (start 54.3506 63.3947) (end 75.4168 63.3947) (width 0.25) (layer B.Cu) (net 20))
 (segment (start 75.4168 63.3947) (end 76.2247 64.2026) (width 0.25) (layer B.Cu) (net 20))
 (segment (start 76.2247 64.2026) (end 76.2247 64.57) (width 0.25) (layer B.Cu) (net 20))
 (segment (start 77.4 64.57) (end 76.2247 64.57) (width 0.25) (layer B.Cu) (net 20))
 (segment (start 52 64.57) (end 53.1753 64.57) (width 0.25) (layer B.Cu) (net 20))
 (segment (start 52 64.57) (end 52 65.7453) (width 0.25) (layer F.Cu) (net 20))
 (segment (start 56.73 71.53) (end 55.5047 71.53) (width 0.25) (layer F.Cu) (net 20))
 (segment (start 55.5047 70.53) (end 55.5047 70.3101) (width 0.25) (layer F.Cu) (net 19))
 (segment (start 55.5047 70.3101) (end 53.6256 68.431) (width 0.25) (layer F.Cu) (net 19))
 (segment (start 53.6256 68.431) (end 53.6256 64.4635) (width 0.25) (layer F.Cu) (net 19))
 (segment (start 53.6256 64.4635) (end 52.3674 63.2053) (width 0.25) (layer F.Cu) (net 19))
 (segment (start 52.3674 63.2053) (end 52 63.2053) (width 0.25) (layer F.Cu) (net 19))
 (segment (start 77.4 62.03) (end 76.2247 62.03) (width 0.25) (layer B.Cu) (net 19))
 (segment (start 52 62.03) (end 53.1753 62.03) (width 0.25) (layer B.Cu) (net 19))
 (segment (start 53.1753 62.03) (end 54.3506 60.8547) (width 0.25) (layer B.Cu) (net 19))
 (segment (start 54.3506 60.8547) (end 75.4168 60.8547) (width 0.25) (layer B.Cu) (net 19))
 (segment (start 75.4168 60.8547) (end 76.2247 61.6626) (width 0.25) (layer B.Cu) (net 19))
 (segment (start 76.2247 61.6626) (end 76.2247 62.03) (width 0.25) (layer B.Cu) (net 19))
 (segment (start 52 62.03) (end 52 63.2053) (width 0.25) (layer F.Cu) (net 19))
 (segment (start 56.73 70.53) (end 55.5047 70.53) (width 0.25) (layer F.Cu) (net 19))
 (segment (start 77.4 59.49) (end 76.2247 59.49) (width 0.25) (layer B.Cu) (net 18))
 (segment (start 52 59.49) (end 53.1753 59.49) (width 0.25) (layer B.Cu) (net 18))
 (segment (start 53.1753 59.49) (end 54.3506 58.3147) (width 0.25) (layer B.Cu) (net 18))
 (segment (start 54.3506 58.3147) (end 75.4168 58.3147) (width 0.25) (layer B.Cu) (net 18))
 (segment (start 75.4168 58.3147) (end 76.2247 59.1226) (width 0.25) (layer B.Cu) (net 18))
 (segment (start 76.2247 59.1226) (end 76.2247 59.49) (width 0.25) (layer B.Cu) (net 18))
 (segment (start 55.5047 69.53) (end 54.0759 68.1012) (width 0.25) (layer F.Cu) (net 18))
 (segment (start 54.0759 68.1012) (end 54.0759 62.3739) (width 0.25) (layer F.Cu) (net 18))
 (segment (start 54.0759 62.3739) (end 52.3673 60.6653) (width 0.25) (layer F.Cu) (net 18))
 (segment (start 52.3673 60.6653) (end 52 60.6653) (width 0.25) (layer F.Cu) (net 18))
 (segment (start 52 59.49) (end 52 60.6653) (width 0.25) (layer F.Cu) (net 18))
 (segment (start 56.73 69.53) (end 55.5047 69.53) (width 0.25) (layer F.Cu) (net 18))
 (segment (start 55.5047 68.53) (end 54.5262 67.5515) (width 0.25) (layer F.Cu) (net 17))
 (segment (start 54.5262 67.5515) (end 54.5262 60.2842) (width 0.25) (layer F.Cu) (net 17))
 (segment (start 54.5262 60.2842) (end 52.3673 58.1253) (width 0.25) (layer F.Cu) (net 17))
 (segment (start 52.3673 58.1253) (end 52 58.1253) (width 0.25) (layer F.Cu) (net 17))
 (segment (start 52 56.95) (end 52 58.1253) (width 0.25) (layer F.Cu) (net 17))
 (segment (start 56.73 68.53) (end 55.5047 68.53) (width 0.25) (layer F.Cu) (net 17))
 (segment (start 77.4 56.95) (end 76.2247 56.95) (width 0.25) (layer B.Cu) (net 17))
 (segment (start 52 56.95) (end 53.1753 56.95) (width 0.25) (layer B.Cu) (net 17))
 (segment (start 53.1753 56.95) (end 54.3506 55.7747) (width 0.25) (layer B.Cu) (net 17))
 (segment (start 54.3506 55.7747) (end 75.4168 55.7747) (width 0.25) (layer B.Cu) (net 17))
 (segment (start 75.4168 55.7747) (end 76.2247 56.5826) (width 0.25) (layer B.Cu) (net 17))
 (segment (start 76.2247 56.5826) (end 76.2247 56.95) (width 0.25) (layer B.Cu) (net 17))
 (segment (start 71.53 66.53) (end 72.7726 66.53) (width 0.25) (layer F.Cu) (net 9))
 (segment (start 72.7726 66.53) (end 73.0325 66.7899) (width 0.25) (layer F.Cu) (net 9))
 (segment (start 74.86 68.4747) (end 74.5614 68.4747) (width 0.25) (layer B.Cu) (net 9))
 (segment (start 74.5614 68.4747) (end 73.0325 66.9458) (width 0.25) (layer B.Cu) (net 9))
 (segment (start 73.0325 66.9458) (end 73.0325 66.7899) (width 0.25) (layer B.Cu) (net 9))
 (segment (start 74.86 69.65) (end 74.86 68.4747) (width 0.25) (layer B.Cu) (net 9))
 (via (at 73.0325 66.7899) (size 0.8) (layers F.Cu B.Cu) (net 9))
 (segment (start 67.63 64.63) (end 68.0717 64.1883) (width 0.25) (layer F.Cu) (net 1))
 (segment (start 68.0717 64.1883) (end 71.9383 64.1883) (width 0.25) (layer F.Cu) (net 1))
 (segment (start 71.9383 64.1883) (end 74.86 67.11) (width 0.25) (layer F.Cu) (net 1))
 (segment (start 66.63 63.4047) (end 72.5194 63.4047) (width 0.25) (layer F.Cu) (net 2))
 (segment (start 72.5194 63.4047) (end 73.6847 64.57) (width 0.25) (layer F.Cu) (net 2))
 (segment (start 74.86 64.57) (end 73.6847 64.57) (width 0.25) (layer F.Cu) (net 2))
 (segment (start 66.63 64.63) (end 66.63 63.4047) (width 0.25) (layer F.Cu) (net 2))
 (segment (start 65.63 63.4047) (end 67.0047 62.03) (width 0.25) (layer F.Cu) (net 3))
 (segment (start 67.0047 62.03) (end 73.6847 62.03) (width 0.25) (layer F.Cu) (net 3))
 (segment (start 74.86 62.03) (end 73.6847 62.03) (width 0.25) (layer F.Cu) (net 3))
 (segment (start 65.63 64.63) (end 65.63 63.4047) (width 0.25) (layer F.Cu) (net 3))
 (segment (start 73.6847 59.49) (end 67.5447 59.49) (width 0.25) (layer F.Cu) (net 5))
 (segment (start 67.5447 59.49) (end 63.63 63.4047) (width 0.25) (layer F.Cu) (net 5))
 (segment (start 74.86 59.49) (end 73.6847 59.49) (width 0.25) (layer F.Cu) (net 5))
 (segment (start 63.63 64.63) (end 63.63 63.4047) (width 0.25) (layer F.Cu) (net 5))
 (segment (start 73.6847 56.95) (end 69.0847 56.95) (width 0.25) (layer F.Cu) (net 6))
 (segment (start 69.0847 56.95) (end 62.63 63.4047) (width 0.25) (layer F.Cu) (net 6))
 (segment (start 74.86 56.95) (end 73.6847 56.95) (width 0.25) (layer F.Cu) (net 6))
 (segment (start 62.63 64.63) (end 62.63 63.4047) (width 0.25) (layer F.Cu) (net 6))
 (segment (start 73.6847 54.41) (end 70.6247 54.41) (width 0.25) (layer F.Cu) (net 7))
 (segment (start 70.6247 54.41) (end 61.63 63.4047) (width 0.25) (layer F.Cu) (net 7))
 (segment (start 74.86 54.41) (end 73.6847 54.41) (width 0.25) (layer F.Cu) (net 7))
 (segment (start 61.63 64.63) (end 61.63 63.4047) (width 0.25) (layer F.Cu) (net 7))
 (segment (start 60.63 63.4047) (end 72.1647 51.87) (width 0.25) (layer F.Cu) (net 8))
 (segment (start 72.1647 51.87) (end 73.6847 51.87) (width 0.25) (layer F.Cu) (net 8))
 (segment (start 74.86 51.87) (end 73.6847 51.87) (width 0.25) (layer F.Cu) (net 8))
 (segment (start 60.63 64.63) (end 60.63 63.4047) (width 0.25) (layer F.Cu) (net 8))
 (segment (start 52 84.89) (end 61.8953 84.89) (width 0.25) (layer F.Cu) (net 25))
 (segment (start 61.8953 84.89) (end 65.63 81.1553) (width 0.25) (layer F.Cu) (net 25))
 (segment (start 65.63 81.1553) (end 70.54 86.0653) (width 0.25) (layer F.Cu) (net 25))
 (segment (start 70.54 86.0653) (end 75.4168 86.0653) (width 0.25) (layer F.Cu) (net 25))
 (segment (start 75.4168 86.0653) (end 76.2247 85.2574) (width 0.25) (layer F.Cu) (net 25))
 (segment (start 76.2247 85.2574) (end 76.2247 84.89) (width 0.25) (layer F.Cu) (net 25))
 (segment (start 77.4 84.89) (end 76.2247 84.89) (width 0.25) (layer F.Cu) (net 25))
 (segment (start 65.63 79.93) (end 65.63 81.1553) (width 0.25) (layer F.Cu) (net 25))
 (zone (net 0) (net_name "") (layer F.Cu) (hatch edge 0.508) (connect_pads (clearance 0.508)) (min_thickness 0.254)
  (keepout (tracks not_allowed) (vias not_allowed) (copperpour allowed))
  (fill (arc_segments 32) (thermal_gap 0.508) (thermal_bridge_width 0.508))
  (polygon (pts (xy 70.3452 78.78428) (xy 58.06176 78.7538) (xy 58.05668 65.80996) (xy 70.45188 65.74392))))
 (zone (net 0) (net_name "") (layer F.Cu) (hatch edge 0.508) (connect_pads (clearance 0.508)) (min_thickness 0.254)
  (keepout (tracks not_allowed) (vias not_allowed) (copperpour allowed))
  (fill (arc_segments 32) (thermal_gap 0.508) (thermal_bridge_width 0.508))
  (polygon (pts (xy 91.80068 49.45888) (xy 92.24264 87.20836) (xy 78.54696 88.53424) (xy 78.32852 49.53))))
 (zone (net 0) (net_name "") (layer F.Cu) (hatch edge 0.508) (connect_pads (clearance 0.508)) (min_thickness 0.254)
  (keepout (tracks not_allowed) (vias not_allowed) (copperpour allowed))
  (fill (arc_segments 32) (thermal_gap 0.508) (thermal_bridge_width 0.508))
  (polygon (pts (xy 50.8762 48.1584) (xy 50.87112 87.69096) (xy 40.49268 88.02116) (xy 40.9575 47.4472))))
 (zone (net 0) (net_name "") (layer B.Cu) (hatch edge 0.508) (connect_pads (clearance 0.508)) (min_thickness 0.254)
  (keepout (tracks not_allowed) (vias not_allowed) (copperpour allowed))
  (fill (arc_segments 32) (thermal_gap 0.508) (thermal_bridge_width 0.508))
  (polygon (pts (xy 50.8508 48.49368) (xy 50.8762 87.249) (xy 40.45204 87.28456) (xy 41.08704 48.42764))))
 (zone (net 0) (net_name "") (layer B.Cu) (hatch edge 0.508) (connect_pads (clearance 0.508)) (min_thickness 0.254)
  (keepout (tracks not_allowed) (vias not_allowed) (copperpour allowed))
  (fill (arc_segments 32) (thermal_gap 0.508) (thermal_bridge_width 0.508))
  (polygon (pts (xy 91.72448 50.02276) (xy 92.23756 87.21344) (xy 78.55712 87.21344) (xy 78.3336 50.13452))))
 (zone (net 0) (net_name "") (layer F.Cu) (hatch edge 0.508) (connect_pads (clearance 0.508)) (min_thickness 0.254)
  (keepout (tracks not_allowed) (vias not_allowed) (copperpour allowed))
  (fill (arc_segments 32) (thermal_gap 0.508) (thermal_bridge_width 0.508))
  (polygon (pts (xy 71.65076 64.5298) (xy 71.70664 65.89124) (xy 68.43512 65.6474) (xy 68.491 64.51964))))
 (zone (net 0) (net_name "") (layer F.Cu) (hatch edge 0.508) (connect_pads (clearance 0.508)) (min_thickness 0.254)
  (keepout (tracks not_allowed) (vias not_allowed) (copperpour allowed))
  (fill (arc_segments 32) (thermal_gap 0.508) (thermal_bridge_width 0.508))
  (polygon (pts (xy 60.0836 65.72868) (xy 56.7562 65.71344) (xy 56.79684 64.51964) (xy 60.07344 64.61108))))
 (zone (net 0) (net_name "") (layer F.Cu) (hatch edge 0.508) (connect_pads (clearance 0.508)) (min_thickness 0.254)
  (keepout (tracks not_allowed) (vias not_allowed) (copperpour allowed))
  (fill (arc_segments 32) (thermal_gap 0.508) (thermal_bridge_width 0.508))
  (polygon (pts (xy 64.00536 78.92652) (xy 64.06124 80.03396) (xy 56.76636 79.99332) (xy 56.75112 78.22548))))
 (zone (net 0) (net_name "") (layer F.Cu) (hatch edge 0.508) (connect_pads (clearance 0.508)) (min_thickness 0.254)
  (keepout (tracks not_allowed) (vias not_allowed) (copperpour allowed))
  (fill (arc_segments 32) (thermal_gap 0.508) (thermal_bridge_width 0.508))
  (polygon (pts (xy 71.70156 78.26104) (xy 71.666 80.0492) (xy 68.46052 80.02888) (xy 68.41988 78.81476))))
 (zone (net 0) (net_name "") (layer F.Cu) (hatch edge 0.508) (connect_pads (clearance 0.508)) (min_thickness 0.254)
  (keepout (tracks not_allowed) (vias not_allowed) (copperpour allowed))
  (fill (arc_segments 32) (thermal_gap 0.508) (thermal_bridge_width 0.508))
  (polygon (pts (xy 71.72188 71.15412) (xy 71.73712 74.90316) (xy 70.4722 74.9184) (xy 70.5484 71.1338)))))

